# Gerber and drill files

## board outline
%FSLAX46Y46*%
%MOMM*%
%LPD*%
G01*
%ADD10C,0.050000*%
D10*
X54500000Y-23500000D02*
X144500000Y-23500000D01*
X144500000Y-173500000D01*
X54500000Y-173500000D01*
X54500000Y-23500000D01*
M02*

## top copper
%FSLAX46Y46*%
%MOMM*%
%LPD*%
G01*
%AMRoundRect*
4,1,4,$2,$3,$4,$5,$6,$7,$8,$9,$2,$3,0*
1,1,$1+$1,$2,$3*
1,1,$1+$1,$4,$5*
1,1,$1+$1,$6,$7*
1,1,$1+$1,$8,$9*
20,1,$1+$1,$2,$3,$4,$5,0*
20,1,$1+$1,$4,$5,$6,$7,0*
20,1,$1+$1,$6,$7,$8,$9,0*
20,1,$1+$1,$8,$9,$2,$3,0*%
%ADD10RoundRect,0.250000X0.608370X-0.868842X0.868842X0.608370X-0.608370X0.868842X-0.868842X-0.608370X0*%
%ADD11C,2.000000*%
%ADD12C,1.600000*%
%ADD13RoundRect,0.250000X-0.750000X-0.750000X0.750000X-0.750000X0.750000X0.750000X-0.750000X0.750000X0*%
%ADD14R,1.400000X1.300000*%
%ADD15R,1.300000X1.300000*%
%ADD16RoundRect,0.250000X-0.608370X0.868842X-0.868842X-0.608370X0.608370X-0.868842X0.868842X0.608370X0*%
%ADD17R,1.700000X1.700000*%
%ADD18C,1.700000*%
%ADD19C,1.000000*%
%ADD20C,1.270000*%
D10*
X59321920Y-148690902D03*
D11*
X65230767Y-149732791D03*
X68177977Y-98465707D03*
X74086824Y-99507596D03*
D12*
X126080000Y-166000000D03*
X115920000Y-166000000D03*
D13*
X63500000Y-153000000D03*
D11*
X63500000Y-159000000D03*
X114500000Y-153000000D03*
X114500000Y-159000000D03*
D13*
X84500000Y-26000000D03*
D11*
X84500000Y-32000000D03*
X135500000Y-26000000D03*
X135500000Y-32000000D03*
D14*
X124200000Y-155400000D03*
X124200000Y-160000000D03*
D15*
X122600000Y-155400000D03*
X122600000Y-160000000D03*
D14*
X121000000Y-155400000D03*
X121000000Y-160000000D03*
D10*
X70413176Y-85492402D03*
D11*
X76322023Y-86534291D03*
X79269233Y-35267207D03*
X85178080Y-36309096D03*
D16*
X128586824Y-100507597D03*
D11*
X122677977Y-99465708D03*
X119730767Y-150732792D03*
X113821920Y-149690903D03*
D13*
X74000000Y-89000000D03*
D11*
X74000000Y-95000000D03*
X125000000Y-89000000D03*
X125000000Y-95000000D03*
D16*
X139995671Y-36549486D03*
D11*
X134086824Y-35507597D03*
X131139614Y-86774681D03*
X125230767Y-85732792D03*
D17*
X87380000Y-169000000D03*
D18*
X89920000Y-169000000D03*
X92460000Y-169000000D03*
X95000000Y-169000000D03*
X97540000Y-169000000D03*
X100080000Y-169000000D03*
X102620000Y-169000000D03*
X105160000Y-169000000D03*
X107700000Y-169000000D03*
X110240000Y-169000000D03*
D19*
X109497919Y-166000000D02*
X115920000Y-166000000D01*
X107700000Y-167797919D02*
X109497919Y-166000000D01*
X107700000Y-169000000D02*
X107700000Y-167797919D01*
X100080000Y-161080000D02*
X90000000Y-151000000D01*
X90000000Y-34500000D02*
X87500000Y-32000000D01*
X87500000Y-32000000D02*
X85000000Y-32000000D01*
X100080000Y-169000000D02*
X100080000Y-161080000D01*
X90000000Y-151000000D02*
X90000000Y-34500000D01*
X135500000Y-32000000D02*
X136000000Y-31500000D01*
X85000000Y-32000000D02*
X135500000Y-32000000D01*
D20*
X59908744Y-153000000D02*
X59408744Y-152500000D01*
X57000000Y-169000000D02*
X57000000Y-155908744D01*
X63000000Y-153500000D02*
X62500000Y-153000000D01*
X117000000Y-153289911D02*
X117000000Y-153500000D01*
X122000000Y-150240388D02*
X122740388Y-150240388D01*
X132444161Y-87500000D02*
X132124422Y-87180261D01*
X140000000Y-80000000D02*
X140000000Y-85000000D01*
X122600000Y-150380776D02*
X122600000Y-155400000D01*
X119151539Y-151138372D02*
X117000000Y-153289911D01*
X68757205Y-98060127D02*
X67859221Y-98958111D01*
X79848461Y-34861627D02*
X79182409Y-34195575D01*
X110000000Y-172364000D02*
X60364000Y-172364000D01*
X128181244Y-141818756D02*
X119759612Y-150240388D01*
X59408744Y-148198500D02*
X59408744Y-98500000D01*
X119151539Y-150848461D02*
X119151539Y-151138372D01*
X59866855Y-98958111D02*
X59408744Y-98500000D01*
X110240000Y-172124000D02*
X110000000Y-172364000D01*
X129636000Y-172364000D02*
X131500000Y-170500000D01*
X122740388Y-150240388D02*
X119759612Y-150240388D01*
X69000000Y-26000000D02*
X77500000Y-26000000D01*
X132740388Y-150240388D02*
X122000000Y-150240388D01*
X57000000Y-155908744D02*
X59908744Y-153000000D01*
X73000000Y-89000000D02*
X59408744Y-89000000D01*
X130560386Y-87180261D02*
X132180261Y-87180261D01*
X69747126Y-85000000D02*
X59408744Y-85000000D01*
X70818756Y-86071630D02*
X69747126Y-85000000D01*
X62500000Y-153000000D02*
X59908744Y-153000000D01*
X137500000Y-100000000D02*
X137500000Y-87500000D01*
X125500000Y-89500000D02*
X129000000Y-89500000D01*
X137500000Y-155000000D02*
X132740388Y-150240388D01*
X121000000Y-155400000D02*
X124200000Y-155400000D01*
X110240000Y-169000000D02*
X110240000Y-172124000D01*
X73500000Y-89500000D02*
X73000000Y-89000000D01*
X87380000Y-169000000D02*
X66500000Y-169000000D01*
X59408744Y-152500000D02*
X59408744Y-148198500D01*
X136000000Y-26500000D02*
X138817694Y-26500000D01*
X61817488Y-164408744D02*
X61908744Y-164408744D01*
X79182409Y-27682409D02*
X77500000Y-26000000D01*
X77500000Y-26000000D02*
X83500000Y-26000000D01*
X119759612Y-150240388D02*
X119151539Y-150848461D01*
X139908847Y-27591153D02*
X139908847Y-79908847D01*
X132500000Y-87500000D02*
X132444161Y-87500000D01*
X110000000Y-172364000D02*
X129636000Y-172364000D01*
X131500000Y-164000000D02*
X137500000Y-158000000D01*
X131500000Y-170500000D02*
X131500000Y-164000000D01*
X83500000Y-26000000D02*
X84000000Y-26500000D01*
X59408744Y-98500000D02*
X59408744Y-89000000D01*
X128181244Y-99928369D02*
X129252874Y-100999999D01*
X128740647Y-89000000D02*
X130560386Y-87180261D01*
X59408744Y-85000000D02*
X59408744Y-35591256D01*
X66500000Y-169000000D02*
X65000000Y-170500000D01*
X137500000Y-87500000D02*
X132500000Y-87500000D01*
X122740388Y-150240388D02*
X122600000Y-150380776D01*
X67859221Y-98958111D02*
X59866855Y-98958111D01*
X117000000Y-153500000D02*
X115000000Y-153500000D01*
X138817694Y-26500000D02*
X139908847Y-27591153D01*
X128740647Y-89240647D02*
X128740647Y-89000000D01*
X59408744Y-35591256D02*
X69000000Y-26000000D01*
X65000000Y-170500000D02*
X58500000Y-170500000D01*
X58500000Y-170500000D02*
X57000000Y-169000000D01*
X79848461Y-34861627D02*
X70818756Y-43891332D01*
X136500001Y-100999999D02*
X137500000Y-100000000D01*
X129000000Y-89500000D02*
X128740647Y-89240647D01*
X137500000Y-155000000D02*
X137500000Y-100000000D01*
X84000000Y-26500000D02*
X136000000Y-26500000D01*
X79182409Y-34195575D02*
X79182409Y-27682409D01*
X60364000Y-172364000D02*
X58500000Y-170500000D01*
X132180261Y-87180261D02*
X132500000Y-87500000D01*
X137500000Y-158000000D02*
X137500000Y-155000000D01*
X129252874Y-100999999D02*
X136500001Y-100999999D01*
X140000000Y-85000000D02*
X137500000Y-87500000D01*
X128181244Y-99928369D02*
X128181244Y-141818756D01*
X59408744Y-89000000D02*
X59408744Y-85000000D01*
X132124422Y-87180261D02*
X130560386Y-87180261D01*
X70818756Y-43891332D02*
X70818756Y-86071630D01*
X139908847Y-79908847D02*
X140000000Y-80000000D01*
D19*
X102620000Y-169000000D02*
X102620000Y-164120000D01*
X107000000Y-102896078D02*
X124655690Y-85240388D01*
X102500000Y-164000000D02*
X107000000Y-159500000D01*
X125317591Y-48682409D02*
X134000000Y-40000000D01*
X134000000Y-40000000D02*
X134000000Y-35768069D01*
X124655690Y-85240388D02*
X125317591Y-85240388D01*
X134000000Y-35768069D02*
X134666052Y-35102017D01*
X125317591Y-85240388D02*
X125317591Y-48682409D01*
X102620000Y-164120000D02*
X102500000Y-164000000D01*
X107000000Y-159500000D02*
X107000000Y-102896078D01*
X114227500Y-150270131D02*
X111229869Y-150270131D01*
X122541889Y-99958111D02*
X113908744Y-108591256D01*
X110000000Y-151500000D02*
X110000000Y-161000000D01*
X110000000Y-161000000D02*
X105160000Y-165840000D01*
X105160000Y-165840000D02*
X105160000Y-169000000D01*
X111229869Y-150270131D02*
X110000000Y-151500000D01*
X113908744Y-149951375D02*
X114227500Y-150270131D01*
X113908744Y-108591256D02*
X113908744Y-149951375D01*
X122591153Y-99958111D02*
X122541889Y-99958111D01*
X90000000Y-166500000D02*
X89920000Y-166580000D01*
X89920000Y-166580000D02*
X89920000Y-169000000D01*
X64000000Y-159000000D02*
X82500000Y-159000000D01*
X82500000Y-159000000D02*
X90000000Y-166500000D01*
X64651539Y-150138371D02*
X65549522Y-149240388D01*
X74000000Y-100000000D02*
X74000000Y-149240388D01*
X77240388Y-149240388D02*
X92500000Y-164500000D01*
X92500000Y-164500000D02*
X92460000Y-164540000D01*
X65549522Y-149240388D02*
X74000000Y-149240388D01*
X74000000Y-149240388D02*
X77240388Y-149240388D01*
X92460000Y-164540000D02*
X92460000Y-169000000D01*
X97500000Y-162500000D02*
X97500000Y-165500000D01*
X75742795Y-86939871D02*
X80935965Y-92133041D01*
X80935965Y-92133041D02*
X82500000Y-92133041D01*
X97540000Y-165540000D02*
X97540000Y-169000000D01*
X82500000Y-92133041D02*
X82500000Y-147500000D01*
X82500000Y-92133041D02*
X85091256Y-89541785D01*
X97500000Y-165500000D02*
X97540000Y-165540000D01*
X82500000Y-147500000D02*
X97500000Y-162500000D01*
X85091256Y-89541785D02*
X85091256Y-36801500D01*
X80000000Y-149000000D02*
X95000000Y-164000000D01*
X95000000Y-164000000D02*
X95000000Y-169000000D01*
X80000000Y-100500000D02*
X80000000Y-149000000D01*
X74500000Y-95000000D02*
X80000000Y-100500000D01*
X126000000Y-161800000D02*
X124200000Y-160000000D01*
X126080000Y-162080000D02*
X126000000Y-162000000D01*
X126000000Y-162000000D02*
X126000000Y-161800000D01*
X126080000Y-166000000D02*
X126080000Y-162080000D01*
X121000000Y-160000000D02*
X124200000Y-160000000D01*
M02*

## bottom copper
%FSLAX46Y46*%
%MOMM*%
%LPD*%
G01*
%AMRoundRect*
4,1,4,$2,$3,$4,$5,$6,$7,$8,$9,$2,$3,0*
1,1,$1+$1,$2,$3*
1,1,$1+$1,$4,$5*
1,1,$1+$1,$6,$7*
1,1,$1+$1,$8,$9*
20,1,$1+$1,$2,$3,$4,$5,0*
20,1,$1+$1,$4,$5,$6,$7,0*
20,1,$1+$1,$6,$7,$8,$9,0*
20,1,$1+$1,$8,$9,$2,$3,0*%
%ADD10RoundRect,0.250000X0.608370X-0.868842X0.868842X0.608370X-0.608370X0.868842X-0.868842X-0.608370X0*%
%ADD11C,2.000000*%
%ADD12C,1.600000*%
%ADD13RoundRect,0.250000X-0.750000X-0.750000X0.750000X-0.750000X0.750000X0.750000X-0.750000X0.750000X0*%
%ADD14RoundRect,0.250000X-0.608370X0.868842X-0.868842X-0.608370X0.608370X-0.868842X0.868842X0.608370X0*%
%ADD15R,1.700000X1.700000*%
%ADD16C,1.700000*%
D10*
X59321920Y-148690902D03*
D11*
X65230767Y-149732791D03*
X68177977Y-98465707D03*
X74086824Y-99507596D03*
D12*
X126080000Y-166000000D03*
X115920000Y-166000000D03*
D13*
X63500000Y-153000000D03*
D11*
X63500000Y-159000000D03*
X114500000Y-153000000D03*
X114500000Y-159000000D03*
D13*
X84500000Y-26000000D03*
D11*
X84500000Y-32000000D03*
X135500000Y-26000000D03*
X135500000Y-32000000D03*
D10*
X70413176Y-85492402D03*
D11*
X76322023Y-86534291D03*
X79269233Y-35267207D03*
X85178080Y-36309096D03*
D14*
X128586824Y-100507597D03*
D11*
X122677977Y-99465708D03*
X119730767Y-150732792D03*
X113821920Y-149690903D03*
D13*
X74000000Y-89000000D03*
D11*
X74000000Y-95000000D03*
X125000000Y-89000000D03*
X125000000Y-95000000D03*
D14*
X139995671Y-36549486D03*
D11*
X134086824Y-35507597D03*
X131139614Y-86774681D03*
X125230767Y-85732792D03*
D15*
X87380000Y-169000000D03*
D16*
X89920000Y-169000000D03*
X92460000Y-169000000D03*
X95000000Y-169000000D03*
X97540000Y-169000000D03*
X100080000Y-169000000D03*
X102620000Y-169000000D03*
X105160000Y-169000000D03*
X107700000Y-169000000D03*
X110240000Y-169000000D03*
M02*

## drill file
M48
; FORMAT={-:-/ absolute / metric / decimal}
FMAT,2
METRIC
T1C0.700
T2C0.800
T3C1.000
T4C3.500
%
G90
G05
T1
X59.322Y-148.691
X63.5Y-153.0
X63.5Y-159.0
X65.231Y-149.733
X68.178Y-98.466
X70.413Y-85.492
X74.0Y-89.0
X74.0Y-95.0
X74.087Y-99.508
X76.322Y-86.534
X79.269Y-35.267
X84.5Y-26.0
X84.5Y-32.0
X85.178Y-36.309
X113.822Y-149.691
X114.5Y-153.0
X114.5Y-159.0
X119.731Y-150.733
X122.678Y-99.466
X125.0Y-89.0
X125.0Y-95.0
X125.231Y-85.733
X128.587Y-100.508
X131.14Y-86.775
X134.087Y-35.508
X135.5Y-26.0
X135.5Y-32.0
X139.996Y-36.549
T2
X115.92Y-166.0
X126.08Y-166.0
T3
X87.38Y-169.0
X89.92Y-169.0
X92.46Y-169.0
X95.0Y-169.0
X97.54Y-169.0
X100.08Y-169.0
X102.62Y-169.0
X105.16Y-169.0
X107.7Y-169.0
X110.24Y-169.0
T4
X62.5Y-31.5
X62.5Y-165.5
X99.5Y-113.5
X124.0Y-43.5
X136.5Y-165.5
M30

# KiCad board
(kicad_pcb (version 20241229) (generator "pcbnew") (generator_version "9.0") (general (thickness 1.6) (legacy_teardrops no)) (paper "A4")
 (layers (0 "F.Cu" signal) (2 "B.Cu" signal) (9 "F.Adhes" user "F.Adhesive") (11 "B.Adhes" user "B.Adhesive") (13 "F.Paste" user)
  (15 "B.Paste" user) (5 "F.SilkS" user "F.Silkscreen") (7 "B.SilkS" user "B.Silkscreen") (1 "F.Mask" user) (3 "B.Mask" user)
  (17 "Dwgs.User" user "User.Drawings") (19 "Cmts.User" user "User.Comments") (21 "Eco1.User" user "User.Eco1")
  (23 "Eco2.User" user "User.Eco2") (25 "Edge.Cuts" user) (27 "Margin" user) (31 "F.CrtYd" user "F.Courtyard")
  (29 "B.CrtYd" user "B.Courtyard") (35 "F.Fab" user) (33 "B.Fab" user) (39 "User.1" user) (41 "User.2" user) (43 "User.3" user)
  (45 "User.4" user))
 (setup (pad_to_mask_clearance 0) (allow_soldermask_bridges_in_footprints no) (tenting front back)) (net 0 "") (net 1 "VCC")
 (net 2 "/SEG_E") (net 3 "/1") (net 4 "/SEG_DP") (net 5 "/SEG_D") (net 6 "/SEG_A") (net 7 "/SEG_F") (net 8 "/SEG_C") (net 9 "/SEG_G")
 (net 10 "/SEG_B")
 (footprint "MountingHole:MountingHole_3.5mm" (layer "F.Cu") (at 62.5 31.5)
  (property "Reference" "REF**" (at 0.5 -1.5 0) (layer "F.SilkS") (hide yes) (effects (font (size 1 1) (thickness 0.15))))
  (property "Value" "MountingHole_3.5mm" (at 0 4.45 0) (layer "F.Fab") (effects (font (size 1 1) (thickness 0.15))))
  (pad "" np_thru_hole circle (at 0 0) (size 3.5 3.5) (drill 3.5) (layers "*.Cu" "*.Mask")))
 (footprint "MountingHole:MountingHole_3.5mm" (layer "F.Cu") (at 124 43.5)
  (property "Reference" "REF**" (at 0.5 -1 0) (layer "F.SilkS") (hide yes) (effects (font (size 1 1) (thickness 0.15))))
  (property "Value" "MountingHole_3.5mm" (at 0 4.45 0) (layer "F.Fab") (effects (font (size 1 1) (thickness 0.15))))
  (pad "" np_thru_hole circle (at 0 0) (size 3.5 3.5) (drill 3.5) (layers "*.Cu" "*.Mask")))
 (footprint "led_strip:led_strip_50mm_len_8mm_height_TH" (layer "F.Cu") (at 66.530724 125.084057 80)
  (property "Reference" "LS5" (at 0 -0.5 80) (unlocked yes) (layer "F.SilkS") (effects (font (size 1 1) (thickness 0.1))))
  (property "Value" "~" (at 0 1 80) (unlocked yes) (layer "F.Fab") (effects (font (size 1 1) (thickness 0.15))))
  (pad "1" thru_hole roundrect (at -24.5 -3 80) (size 2 2) (drill 0.7) (layers "*.Cu" "*.Mask") (remove_unused_layers no)
   (roundrect_rratio 0.125) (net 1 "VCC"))
  (pad "2" thru_hole circle (at -24.5 3 80) (size 2 2) (drill 0.7) (layers "*.Cu" "*.Mask") (remove_unused_layers no) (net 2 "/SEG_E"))
  (pad "3" thru_hole circle (at 26.5 -3 80) (size 2 2) (drill 0.7) (layers "*.Cu" "*.Mask") (remove_unused_layers no) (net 1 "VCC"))
  (pad "4" thru_hole circle (at 26.5 3 80) (size 2 2) (drill 0.7) (layers "*.Cu" "*.Mask") (remove_unused_layers no) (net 2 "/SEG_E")))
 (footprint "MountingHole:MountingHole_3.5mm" (layer "F.Cu") (at 99.5 113.5)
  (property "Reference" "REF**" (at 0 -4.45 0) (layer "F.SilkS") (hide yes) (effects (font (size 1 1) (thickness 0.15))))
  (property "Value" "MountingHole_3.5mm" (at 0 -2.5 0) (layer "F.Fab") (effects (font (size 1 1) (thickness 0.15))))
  (pad "" np_thru_hole circle (at 0 0) (size 3.5 3.5) (drill 3.5) (layers "*.Cu" "*.Mask")))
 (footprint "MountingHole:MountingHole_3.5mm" (layer "F.Cu") (at 136.5 165.5)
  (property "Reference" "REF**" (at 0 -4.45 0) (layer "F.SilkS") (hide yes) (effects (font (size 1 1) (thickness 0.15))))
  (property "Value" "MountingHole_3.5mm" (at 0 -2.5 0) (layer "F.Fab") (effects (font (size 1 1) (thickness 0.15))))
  (pad "" np_thru_hole circle (at 0 0) (size 3.5 3.5) (drill 3.5) (layers "*.Cu" "*.Mask")))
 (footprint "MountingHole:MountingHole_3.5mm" (layer "F.Cu") (at 62.5 165.5)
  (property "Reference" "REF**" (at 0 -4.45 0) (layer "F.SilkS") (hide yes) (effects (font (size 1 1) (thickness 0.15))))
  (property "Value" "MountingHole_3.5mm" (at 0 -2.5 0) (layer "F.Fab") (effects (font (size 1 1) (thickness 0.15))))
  (pad "" np_thru_hole circle (at 0 0) (size 3.5 3.5) (drill 3.5) (layers "*.Cu" "*.Mask")))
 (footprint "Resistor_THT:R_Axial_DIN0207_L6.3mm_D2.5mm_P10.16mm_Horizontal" (layer "F.Cu") (at 126.08 166 180)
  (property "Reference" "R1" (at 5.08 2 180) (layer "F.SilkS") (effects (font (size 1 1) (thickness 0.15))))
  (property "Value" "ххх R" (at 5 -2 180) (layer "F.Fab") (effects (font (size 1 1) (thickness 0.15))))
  (pad "1" thru_hole circle (at 0 0 180) (size 1.6 1.6) (drill 0.8) (layers "*.Cu" "*.Mask") (remove_unused_layers no) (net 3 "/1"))
  (pad "2" thru_hole circle (at 10.16 0 180) (size 1.6 1.6) (drill 0.8) (layers "*.Cu" "*.Mask") (remove_unused_layers no) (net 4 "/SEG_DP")))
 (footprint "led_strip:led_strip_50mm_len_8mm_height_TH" (layer "F.Cu") (at 88 156)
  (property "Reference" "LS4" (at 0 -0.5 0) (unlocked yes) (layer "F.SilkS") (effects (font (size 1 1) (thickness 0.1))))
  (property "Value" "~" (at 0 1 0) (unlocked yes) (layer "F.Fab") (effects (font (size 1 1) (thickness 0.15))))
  (pad "1" thru_hole roundrect (at -24.5 -3) (size 2 2) (drill 0.7) (layers "*.Cu" "*.Mask") (remove_unused_layers no)
   (roundrect_rratio 0.125) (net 1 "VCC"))
  (pad "2" thru_hole circle (at -24.5 3) (size 2 2) (drill 0.7) (layers "*.Cu" "*.Mask") (remove_unused_layers no) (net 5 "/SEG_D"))
  (pad "3" thru_hole circle (at 26.5 -3) (size 2 2) (drill 0.7) (layers "*.Cu" "*.Mask") (remove_unused_layers no) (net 1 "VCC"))
  (pad "4" thru_hole circle (at 26.5 3) (size 2 2) (drill 0.7) (layers "*.Cu" "*.Mask") (remove_unused_layers no) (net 5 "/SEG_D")))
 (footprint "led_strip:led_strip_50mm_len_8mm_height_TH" (layer "F.Cu") (at 109 29)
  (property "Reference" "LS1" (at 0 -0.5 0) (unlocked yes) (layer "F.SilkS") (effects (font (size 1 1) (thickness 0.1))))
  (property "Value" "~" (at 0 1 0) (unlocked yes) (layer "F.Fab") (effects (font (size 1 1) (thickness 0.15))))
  (pad "1" thru_hole roundrect (at -24.5 -3) (size 2 2) (drill 0.7) (layers "*.Cu" "*.Mask") (remove_unused_layers no)
   (roundrect_rratio 0.125) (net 1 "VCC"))
  (pad "2" thru_hole circle (at -24.5 3) (size 2 2) (drill 0.7) (layers "*.Cu" "*.Mask") (remove_unused_layers no) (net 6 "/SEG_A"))
  (pad "3" thru_hole circle (at 26.5 -3) (size 2 2) (drill 0.7) (layers "*.Cu" "*.Mask") (remove_unused_layers no) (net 1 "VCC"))
  (pad "4" thru_hole circle (at 26.5 3) (size 2 2) (drill 0.7) (layers "*.Cu" "*.Mask") (remove_unused_layers no) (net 6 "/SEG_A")))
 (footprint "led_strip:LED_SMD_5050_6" (layer "F.Cu") (at 122.6 157.6 -90)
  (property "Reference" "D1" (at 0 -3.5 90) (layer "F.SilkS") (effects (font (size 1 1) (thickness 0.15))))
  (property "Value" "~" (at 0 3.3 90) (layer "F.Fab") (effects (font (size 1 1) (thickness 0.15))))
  (pad "1" smd rect (at -2.2 -1.6 270) (size 1.3 1.4) (layers "F.Cu" "F.Mask" "F.Paste") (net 1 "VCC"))
  (pad "2" smd rect (at 2.4 -1.6 270) (size 1.3 1.4) (layers "F.Cu" "F.Mask" "F.Paste") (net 3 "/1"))
  (pad "3" smd rect (at -2.2 0) (size 1.3 1.3) (layers "F.Cu" "F.Mask" "F.Paste") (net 1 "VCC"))
  (pad "4" smd rect (at 2.4 0) (size 1.3 1.3) (layers "F.Cu" "F.Mask" "F.Paste") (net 3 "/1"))
  (pad "5" smd rect (at -2.2 1.6 270) (size 1.3 1.4) (layers "F.Cu" "F.Mask" "F.Paste") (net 1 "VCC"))
  (pad "6" smd rect (at 2.4 1.6 270) (size 1.3 1.4) (layers "F.Cu" "F.Mask" "F.Paste") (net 3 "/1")))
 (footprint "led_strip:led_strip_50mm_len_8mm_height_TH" (layer "F.Cu") (at 77.62198 61.885557 80)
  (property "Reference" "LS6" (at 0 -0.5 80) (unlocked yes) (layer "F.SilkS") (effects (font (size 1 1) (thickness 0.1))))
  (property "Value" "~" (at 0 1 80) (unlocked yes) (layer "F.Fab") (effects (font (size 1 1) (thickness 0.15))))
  (pad "1" thru_hole roundrect (at -24.5 -3 80) (size 2 2) (drill 0.7) (layers "*.Cu" "*.Mask") (remove_unused_layers no)
   (roundrect_rratio 0.125) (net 1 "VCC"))
  (pad "2" thru_hole circle (at -24.5 3 80) (size 2 2) (drill 0.7) (layers "*.Cu" "*.Mask") (remove_unused_layers no) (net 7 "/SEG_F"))
  (pad "3" thru_hole circle (at 26.5 -3 80) (size 2 2) (drill 0.7) (layers "*.Cu" "*.Mask") (remove_unused_layers no) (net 1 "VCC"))
  (pad "4" thru_hole circle (at 26.5 3 80) (size 2 2) (drill 0.7) (layers "*.Cu" "*.Mask") (remove_unused_layers no) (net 7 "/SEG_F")))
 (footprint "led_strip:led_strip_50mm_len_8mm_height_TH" (layer "F.Cu") (at 121.37802 124.114442 -100)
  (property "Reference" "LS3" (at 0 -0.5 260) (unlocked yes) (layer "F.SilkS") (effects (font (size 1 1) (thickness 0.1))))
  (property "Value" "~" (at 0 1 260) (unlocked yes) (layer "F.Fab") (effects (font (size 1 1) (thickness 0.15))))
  (pad "1" thru_hole roundrect (at -24.5 -3 260) (size 2 2) (drill 0.7) (layers "*.Cu" "*.Mask") (remove_unused_layers no)
   (roundrect_rratio 0.125) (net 1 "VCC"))
  (pad "2" thru_hole circle (at -24.5 3 260) (size 2 2) (drill 0.7) (layers "*.Cu" "*.Mask") (remove_unused_layers no) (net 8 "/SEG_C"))
  (pad "3" thru_hole circle (at 26.5 -3 260) (size 2 2) (drill 0.7) (layers "*.Cu" "*.Mask") (remove_unused_layers no) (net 1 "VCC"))
  (pad "4" thru_hole circle (at 26.5 3 260) (size 2 2) (drill 0.7) (layers "*.Cu" "*.Mask") (remove_unused_layers no) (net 8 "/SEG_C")))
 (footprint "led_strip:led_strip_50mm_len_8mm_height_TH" (layer "F.Cu") (at 98.5 92)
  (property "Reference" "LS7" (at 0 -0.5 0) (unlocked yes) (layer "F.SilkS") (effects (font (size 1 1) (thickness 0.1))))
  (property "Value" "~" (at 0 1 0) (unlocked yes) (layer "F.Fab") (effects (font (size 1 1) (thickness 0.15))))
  (pad "1" thru_hole roundrect (at -24.5 -3) (size 2 2) (drill 0.7) (layers "*.Cu" "*.Mask") (remove_unused_layers no)
   (roundrect_rratio 0.125) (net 1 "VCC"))
  (pad "2" thru_hole circle (at -24.5 3) (size 2 2) (drill 0.7) (layers "*.Cu" "*.Mask") (remove_unused_layers no) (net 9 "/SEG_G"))
  (pad "3" thru_hole circle (at 26.5 -3) (size 2 2) (drill 0.7) (layers "*.Cu" "*.Mask") (remove_unused_layers no) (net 1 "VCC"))
  (pad "4" thru_hole circle (at 26.5 3) (size 2 2) (drill 0.7) (layers "*.Cu" "*.Mask") (remove_unused_layers no) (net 9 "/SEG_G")))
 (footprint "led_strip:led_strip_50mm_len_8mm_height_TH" (layer "F.Cu") (at 132.786867 60.156331 -100)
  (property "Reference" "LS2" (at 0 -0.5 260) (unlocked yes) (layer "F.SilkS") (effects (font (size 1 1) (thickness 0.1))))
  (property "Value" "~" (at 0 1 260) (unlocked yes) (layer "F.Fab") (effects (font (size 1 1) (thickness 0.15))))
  (pad "1" thru_hole roundrect (at -24.5 -3 260) (size 2 2) (drill 0.7) (layers "*.Cu" "*.Mask") (remove_unused_layers no)
   (roundrect_rratio 0.125) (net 1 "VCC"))
  (pad "2" thru_hole circle (at -24.5 3 260) (size 2 2) (drill 0.7) (layers "*.Cu" "*.Mask") (remove_unused_layers no) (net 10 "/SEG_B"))
  (pad "3" thru_hole circle (at 26.5 -3 260) (size 2 2) (drill 0.7) (layers "*.Cu" "*.Mask") (remove_unused_layers no) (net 1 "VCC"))
  (pad "4" thru_hole circle (at 26.5 3 260) (size 2 2) (drill 0.7) (layers "*.Cu" "*.Mask") (remove_unused_layers no) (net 10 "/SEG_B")))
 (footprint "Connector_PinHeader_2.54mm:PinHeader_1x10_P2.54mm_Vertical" (layer "F.Cu") (at 87.38 169 90)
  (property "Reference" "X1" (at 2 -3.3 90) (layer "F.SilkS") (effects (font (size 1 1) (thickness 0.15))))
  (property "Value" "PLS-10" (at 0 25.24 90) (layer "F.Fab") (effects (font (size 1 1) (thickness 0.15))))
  (pad "1" thru_hole rect (at 0 0 90) (size 1.7 1.7) (drill 1) (layers "*.Cu" "*.Mask") (remove_unused_layers no) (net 1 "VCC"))
  (pad "2" thru_hole circle (at 0 2.54 90) (size 1.7 1.7) (drill 1) (layers "*.Cu" "*.Mask") (remove_unused_layers no) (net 5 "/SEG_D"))
  (pad "3" thru_hole circle (at 0 5.08 90) (size 1.7 1.7) (drill 1) (layers "*.Cu" "*.Mask") (remove_unused_layers no) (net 2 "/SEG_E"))
  (pad "4" thru_hole circle (at 0 7.62 90) (size 1.7 1.7) (drill 1) (layers "*.Cu" "*.Mask") (remove_unused_layers no) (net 9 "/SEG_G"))
  (pad "5" thru_hole circle (at 0 10.16 90) (size 1.7 1.7) (drill 1) (layers "*.Cu" "*.Mask") (remove_unused_layers no) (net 7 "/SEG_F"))
  (pad "6" thru_hole circle (at 0 12.7 90) (size 1.7 1.7) (drill 1) (layers "*.Cu" "*.Mask") (remove_unused_layers no) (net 6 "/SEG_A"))
  (pad "7" thru_hole circle (at 0 15.24 90) (size 1.7 1.7) (drill 1) (layers "*.Cu" "*.Mask") (remove_unused_layers no) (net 10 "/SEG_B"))
  (pad "8" thru_hole circle (at 0 17.78 90) (size 1.7 1.7) (drill 1) (layers "*.Cu" "*.Mask") (remove_unused_layers no) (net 8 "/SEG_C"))
  (pad "9" thru_hole circle (at 0 20.32 90) (size 1.7 1.7) (drill 1) (layers "*.Cu" "*.Mask") (remove_unused_layers no) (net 4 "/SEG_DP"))
  (pad "10" thru_hole circle (at 0 22.86 90) (size 1.7 1.7) (drill 1) (layers "*.Cu" "*.Mask") (remove_unused_layers no) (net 1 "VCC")))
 (gr_rect (start 54.5 23.5) (end 144.5 173.5) (stroke (width 0.05) (type default)) (fill no) (layer "Edge.Cuts"))
 (segment (start 109.497919 166) (end 115.92 166) (width 1) (layer "F.Cu") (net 4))
 (segment (start 107.7 167.797919) (end 109.497919 166) (width 1) (layer "F.Cu") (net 4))
 (segment (start 107.7 169) (end 107.7 167.797919) (width 1) (layer "F.Cu") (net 4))
 (segment (start 100.08 161.08) (end 90 151) (width 1) (layer "F.Cu") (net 6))
 (segment (start 90 34.5) (end 87.5 32) (width 1) (layer "F.Cu") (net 6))
 (segment (start 87.5 32) (end 85 32) (width 1) (layer "F.Cu") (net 6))
 (segment (start 100.08 169) (end 100.08 161.08) (width 1) (layer "F.Cu") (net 6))
 (segment (start 90 151) (end 90 34.5) (width 1) (layer "F.Cu") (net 6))
 (segment (start 135.5 32) (end 136 31.5) (width 1) (layer "F.Cu") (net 6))
 (segment (start 85 32) (end 135.5 32) (width 1) (layer "F.Cu") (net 6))
 (segment (start 59.908744 153) (end 59.408744 152.5) (width 1.27) (layer "F.Cu") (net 1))
 (segment (start 57 169) (end 57 155.908744) (width 1.27) (layer "F.Cu") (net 1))
 (segment (start 63 153.5) (end 62.5 153) (width 1.27) (layer "F.Cu") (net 1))
 (segment (start 117 153.289911) (end 117 153.5) (width 1.27) (layer "F.Cu") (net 1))
 (segment (start 122 150.240388) (end 122.740388 150.240388) (width 1.27) (layer "F.Cu") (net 1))
 (segment (start 132.444161 87.5) (end 132.124422 87.180261) (width 1.27) (layer "F.Cu") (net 1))
 (segment (start 140 80) (end 140 85) (width 1.27) (layer "F.Cu") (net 1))
 (segment (start 122.6 150.380776) (end 122.6 155.4) (width 1.27) (layer "F.Cu") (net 1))
 (segment (start 119.151539 151.138372) (end 117 153.289911) (width 1.27) (layer "F.Cu") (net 1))
 (segment (start 68.757205 98.060127) (end 67.859221 98.958111) (width 1.27) (layer "F.Cu") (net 1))
 (segment (start 79.848461 34.861627) (end 79.182409 34.195575) (width 1.27) (layer "F.Cu") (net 1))
 (segment (start 110 172.364) (end 60.364 172.364) (width 1.27) (layer "F.Cu") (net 1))
 (segment (start 128.181244 141.818756) (end 119.759612 150.240388) (width 1.27) (layer "F.Cu") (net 1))
 (segment (start 59.408744 148.1985) (end 59.408744 98.5) (width 1.27) (layer "F.Cu") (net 1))
 (segment (start 119.151539 150.848461) (end 119.151539 151.138372) (width 1.27) (layer "F.Cu") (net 1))
 (segment (start 59.866855 98.958111) (end 59.408744 98.5) (width 1.27) (layer "F.Cu") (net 1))
 (segment (start 110.24 172.124) (end 110 172.364) (width 1.27) (layer "F.Cu") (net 1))
 (segment (start 129.636 172.364) (end 131.5 170.5) (width 1.27) (layer "F.Cu") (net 1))
 (segment (start 122.740388 150.240388) (end 119.759612 150.240388) (width 1.27) (layer "F.Cu") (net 1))
 (segment (start 69 26) (end 77.5 26) (width 1.27) (layer "F.Cu") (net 1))
 (segment (start 132.740388 150.240388) (end 122 150.240388) (width 1.27) (layer "F.Cu") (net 1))
 (segment (start 57 155.908744) (end 59.908744 153) (width 1.27) (layer "F.Cu") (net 1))
 (segment (start 73 89) (end 59.408744 89) (width 1.27) (layer "F.Cu") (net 1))
 (segment (start 130.560386 87.180261) (end 132.180261 87.180261) (width 1.27) (layer "F.Cu") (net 1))
 (segment (start 69.747126 85) (end 59.408744 85) (width 1.27) (layer "F.Cu") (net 1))
 (segment (start 70.818756 86.07163) (end 69.747126 85) (width 1.27) (layer "F.Cu") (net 1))
 (segment (start 62.5 153) (end 59.908744 153) (width 1.27) (layer "F.Cu") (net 1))
 (segment (start 137.5 100) (end 137.5 87.5) (width 1.27) (layer "F.Cu") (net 1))
 (segment (start 125.5 89.5) (end 129 89.5) (width 1.27) (layer "F.Cu") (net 1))
 (segment (start 137.5 155) (end 132.740388 150.240388) (width 1.27) (layer "F.Cu") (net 1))
 (segment (start 121 155.4) (end 124.2 155.4) (width 1.27) (layer "F.Cu") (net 1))
 (segment (start 110.24 169) (end 110.24 172.124) (width 1.27) (layer "F.Cu") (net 1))
 (segment (start 73.5 89.5) (end 73 89) (width 1.27) (layer "F.Cu") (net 1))
 (segment (start 87.38 169) (end 66.5 169) (width 1.27) (layer "F.Cu") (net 1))
 (segment (start 59.408744 152.5) (end 59.408744 148.1985) (width 1.27) (layer "F.Cu") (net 1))
 (segment (start 136 26.5) (end 138.817694 26.5) (width 1.27) (layer "F.Cu") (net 1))
 (segment (start 61.817488 164.408744) (end 61.908744 164.408744) (width 1.27) (layer "F.Cu") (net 1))
 (segment (start 79.182409 27.682409) (end 77.5 26) (width 1.27) (layer "F.Cu") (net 1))
 (segment (start 77.5 26) (end 83.5 26) (width 1.27) (layer "F.Cu") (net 1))
 (segment (start 119.759612 150.240388) (end 119.151539 150.848461) (width 1.27) (layer "F.Cu") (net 1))
 (segment (start 139.908847 27.591153) (end 139.908847 79.908847) (width 1.27) (layer "F.Cu") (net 1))
 (segment (start 132.5 87.5) (end 132.444161 87.5) (width 1.27) (layer "F.Cu") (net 1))
 (segment (start 110 172.364) (end 129.636 172.364) (width 1.27) (layer "F.Cu") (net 1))
 (segment (start 131.5 164) (end 137.5 158) (width 1.27) (layer "F.Cu") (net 1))
 (segment (start 131.5 170.5) (end 131.5 164) (width 1.27) (layer "F.Cu") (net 1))
 (segment (start 83.5 26) (end 84 26.5) (width 1.27) (layer "F.Cu") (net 1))
 (segment (start 59.408744 98.5) (end 59.408744 89) (width 1.27) (layer "F.Cu") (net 1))
 (segment (start 128.181244 99.928369) (end 129.252874 100.999999) (width 1.27) (layer "F.Cu") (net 1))
 (segment (start 128.740647 89) (end 130.560386 87.180261) (width 1.27) (layer "F.Cu") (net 1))
 (segment (start 59.408744 85) (end 59.408744 35.591256) (width 1.27) (layer "F.Cu") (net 1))
 (segment (start 66.5 169) (end 65 170.5) (width 1.27) (layer "F.Cu") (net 1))
 (segment (start 137.5 87.5) (end 132.5 87.5) (width 1.27) (layer "F.Cu") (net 1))
 (segment (start 122.740388 150.240388) (end 122.6 150.380776) (width 1.27) (layer "F.Cu") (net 1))
 (segment (start 67.859221 98.958111) (end 59.866855 98.958111) (width 1.27) (layer "F.Cu") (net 1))
 (segment (start 117 153.5) (end 115 153.5) (width 1.27) (layer "F.Cu") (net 1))
 (segment (start 138.817694 26.5) (end 139.908847 27.591153) (width 1.27) (layer "F.Cu") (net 1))
 (segment (start 128.740647 89.240647) (end 128.740647 89) (width 1.27) (layer "F.Cu") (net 1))
 (segment (start 59.408744 35.591256) (end 69 26) (width 1.27) (layer "F.Cu") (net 1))
 (segment (start 65 170.5) (end 58.5 170.5) (width 1.27) (layer "F.Cu") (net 1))
 (segment (start 58.5 170.5) (end 57 169) (width 1.27) (layer "F.Cu") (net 1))
 (segment (start 79.848461 34.861627) (end 70.818756 43.891332) (width 1.27) (layer "F.Cu") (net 1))
 (segment (start 136.500001 100.999999) (end 137.5 100) (width 1.27) (layer "F.Cu") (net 1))
 (segment (start 129 89.5) (end 128.740647 89.240647) (width 1.27) (layer "F.Cu") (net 1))
 (segment (start 137.5 155) (end 137.5 100) (width 1.27) (layer "F.Cu") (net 1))
 (segment (start 84 26.5) (end 136 26.5) (width 1.27) (layer "F.Cu") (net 1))
 (segment (start 79.182409 34.195575) (end 79.182409 27.682409) (width 1.27) (layer "F.Cu") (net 1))
 (segment (start 60.364 172.364) (end 58.5 170.5) (width 1.27) (layer "F.Cu") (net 1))
 (segment (start 132.180261 87.180261) (end 132.5 87.5) (width 1.27) (layer "F.Cu") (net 1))
 (segment (start 137.5 158) (end 137.5 155) (width 1.27) (layer "F.Cu") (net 1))
 (segment (start 129.252874 100.999999) (end 136.500001 100.999999) (width 1.27) (layer "F.Cu") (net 1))
 (segment (start 140 85) (end 137.5 87.5) (width 1.27) (layer "F.Cu") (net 1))
 (segment (start 128.181244 99.928369) (end 128.181244 141.818756) (width 1.27) (layer "F.Cu") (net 1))
 (segment (start 59.408744 89) (end 59.408744 85) (width 1.27) (layer "F.Cu") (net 1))
 (segment (start 132.124422 87.180261) (end 130.560386 87.180261) (width 1.27) (layer "F.Cu") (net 1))
 (segment (start 70.818756 43.891332) (end 70.818756 86.07163) (width 1.27) (layer "F.Cu") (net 1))
 (segment (start 139.908847 79.908847) (end 140 80) (width 1.27) (layer "F.Cu") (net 1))
 (segment (start 102.62 169) (end 102.62 164.12) (width 1) (layer "F.Cu") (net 10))
 (segment (start 107 102.896078) (end 124.65569 85.240388) (width 1) (layer "F.Cu") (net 10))
 (segment (start 102.5 164) (end 107 159.5) (width 1) (layer "F.Cu") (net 10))
 (segment (start 125.317591 48.682409) (end 134 40) (width 1) (layer "F.Cu") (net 10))
 (segment (start 134 40) (end 134 35.768069) (width 1) (layer "F.Cu") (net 10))
 (segment (start 124.65569 85.240388) (end 125.317591 85.240388) (width 1) (layer "F.Cu") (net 10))
 (segment (start 134 35.768069) (end 134.666052 35.102017) (width 1) (layer "F.Cu") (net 10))
 (segment (start 125.317591 85.240388) (end 125.317591 48.682409) (width 1) (layer "F.Cu") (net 10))
 (segment (start 102.62 164.12) (end 102.5 164) (width 1) (layer "F.Cu") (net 10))
 (segment (start 107 159.5) (end 107 102.896078) (width 1) (layer "F.Cu") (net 10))
 (segment (start 114.2275 150.270131) (end 111.229869 150.270131) (width 1) (layer "F.Cu") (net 8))
 (segment (start 122.541889 99.958111) (end 113.908744 108.591256) (width 1) (layer "F.Cu") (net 8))
 (segment (start 110 151.5) (end 110 161) (width 1) (layer "F.Cu") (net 8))
 (segment (start 110 161) (end 105.16 165.84) (width 1) (layer "F.Cu") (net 8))
 (segment (start 105.16 165.84) (end 105.16 169) (width 1) (layer "F.Cu") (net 8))
 (segment (start 111.229869 150.270131) (end 110 151.5) (width 1) (layer "F.Cu") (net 8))
 (segment (start 113.908744 149.951375) (end 114.2275 150.270131) (width 1) (layer "F.Cu") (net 8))
 (segment (start 113.908744 108.591256) (end 113.908744 149.951375) (width 1) (layer "F.Cu") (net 8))
 (segment (start 122.591153 99.958111) (end 122.541889 99.958111) (width 1) (layer "F.Cu") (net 8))
 (segment (start 90 166.5) (end 89.92 166.58) (width 1) (layer "F.Cu") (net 5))
 (segment (start 89.92 166.58) (end 89.92 169) (width 1) (layer "F.Cu") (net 5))
 (segment (start 64 159) (end 82.5 159) (width 1) (layer "F.Cu") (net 5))
 (segment (start 82.5 159) (end 90 166.5) (width 1) (layer "F.Cu") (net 5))
 (segment (start 64.651539 150.138371) (end 65.549522 149.240388) (width 1) (layer "F.Cu") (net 2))
 (segment (start 74 100) (end 74 149.240388) (width 1) (layer "F.Cu") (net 2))
 (segment (start 77.240388 149.240388) (end 92.5 164.5) (width 1) (layer "F.Cu") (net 2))
 (segment (start 92.5 164.5) (end 92.46 164.54) (width 1) (layer "F.Cu") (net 2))
 (segment (start 65.549522 149.240388) (end 74 149.240388) (width 1) (layer "F.Cu") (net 2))
 (segment (start 74 149.240388) (end 77.240388 149.240388) (width 1) (layer "F.Cu") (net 2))
 (segment (start 92.46 164.54) (end 92.46 169) (width 1) (layer "F.Cu") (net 2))
 (segment (start 97.5 162.5) (end 97.5 165.5) (width 1) (layer "F.Cu") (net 7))
 (segment (start 75.742795 86.939871) (end 80.935965 92.133041) (width 1) (layer "F.Cu") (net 7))
 (segment (start 80.935965 92.133041) (end 82.5 92.133041) (width 1) (layer "F.Cu") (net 7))
 (segment (start 97.54 165.54) (end 97.54 169) (width 1) (layer "F.Cu") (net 7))
 (segment (start 82.5 92.133041) (end 82.5 147.5) (width 1) (layer "F.Cu") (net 7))
 (segment (start 82.5 92.133041) (end 85.091256 89.541785) (width 1) (layer "F.Cu") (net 7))
 (segment (start 97.5 165.5) (end 97.54 165.54) (width 1) (layer "F.Cu") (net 7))
 (segment (start 82.5 147.5) (end 97.5 162.5) (width 1) (layer "F.Cu") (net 7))
 (segment (start 85.091256 89.541785) (end 85.091256 36.8015) (width 1) (layer "F.Cu") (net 7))
 (segment (start 80 149) (end 95 164) (width 1) (layer "F.Cu") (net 9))
 (segment (start 95 164) (end 95 169) (width 1) (layer "F.Cu") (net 9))
 (segment (start 80 100.5) (end 80 149) (width 1) (layer "F.Cu") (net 9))
 (segment (start 74.5 95) (end 80 100.5) (width 1) (layer "F.Cu") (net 9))
 (segment (start 126 161.8) (end 124.2 160) (width 1) (layer "F.Cu") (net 3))
 (segment (start 126.08 162.08) (end 126 162) (width 1) (layer "F.Cu") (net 3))
 (segment (start 126 162) (end 126 161.8) (width 1) (layer "F.Cu") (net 3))
 (segment (start 126.08 166) (end 126.08 162.08) (width 1) (layer "F.Cu") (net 3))
 (segment (start 121 160) (end 124.2 160) (width 1) (layer "F.Cu") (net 3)))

